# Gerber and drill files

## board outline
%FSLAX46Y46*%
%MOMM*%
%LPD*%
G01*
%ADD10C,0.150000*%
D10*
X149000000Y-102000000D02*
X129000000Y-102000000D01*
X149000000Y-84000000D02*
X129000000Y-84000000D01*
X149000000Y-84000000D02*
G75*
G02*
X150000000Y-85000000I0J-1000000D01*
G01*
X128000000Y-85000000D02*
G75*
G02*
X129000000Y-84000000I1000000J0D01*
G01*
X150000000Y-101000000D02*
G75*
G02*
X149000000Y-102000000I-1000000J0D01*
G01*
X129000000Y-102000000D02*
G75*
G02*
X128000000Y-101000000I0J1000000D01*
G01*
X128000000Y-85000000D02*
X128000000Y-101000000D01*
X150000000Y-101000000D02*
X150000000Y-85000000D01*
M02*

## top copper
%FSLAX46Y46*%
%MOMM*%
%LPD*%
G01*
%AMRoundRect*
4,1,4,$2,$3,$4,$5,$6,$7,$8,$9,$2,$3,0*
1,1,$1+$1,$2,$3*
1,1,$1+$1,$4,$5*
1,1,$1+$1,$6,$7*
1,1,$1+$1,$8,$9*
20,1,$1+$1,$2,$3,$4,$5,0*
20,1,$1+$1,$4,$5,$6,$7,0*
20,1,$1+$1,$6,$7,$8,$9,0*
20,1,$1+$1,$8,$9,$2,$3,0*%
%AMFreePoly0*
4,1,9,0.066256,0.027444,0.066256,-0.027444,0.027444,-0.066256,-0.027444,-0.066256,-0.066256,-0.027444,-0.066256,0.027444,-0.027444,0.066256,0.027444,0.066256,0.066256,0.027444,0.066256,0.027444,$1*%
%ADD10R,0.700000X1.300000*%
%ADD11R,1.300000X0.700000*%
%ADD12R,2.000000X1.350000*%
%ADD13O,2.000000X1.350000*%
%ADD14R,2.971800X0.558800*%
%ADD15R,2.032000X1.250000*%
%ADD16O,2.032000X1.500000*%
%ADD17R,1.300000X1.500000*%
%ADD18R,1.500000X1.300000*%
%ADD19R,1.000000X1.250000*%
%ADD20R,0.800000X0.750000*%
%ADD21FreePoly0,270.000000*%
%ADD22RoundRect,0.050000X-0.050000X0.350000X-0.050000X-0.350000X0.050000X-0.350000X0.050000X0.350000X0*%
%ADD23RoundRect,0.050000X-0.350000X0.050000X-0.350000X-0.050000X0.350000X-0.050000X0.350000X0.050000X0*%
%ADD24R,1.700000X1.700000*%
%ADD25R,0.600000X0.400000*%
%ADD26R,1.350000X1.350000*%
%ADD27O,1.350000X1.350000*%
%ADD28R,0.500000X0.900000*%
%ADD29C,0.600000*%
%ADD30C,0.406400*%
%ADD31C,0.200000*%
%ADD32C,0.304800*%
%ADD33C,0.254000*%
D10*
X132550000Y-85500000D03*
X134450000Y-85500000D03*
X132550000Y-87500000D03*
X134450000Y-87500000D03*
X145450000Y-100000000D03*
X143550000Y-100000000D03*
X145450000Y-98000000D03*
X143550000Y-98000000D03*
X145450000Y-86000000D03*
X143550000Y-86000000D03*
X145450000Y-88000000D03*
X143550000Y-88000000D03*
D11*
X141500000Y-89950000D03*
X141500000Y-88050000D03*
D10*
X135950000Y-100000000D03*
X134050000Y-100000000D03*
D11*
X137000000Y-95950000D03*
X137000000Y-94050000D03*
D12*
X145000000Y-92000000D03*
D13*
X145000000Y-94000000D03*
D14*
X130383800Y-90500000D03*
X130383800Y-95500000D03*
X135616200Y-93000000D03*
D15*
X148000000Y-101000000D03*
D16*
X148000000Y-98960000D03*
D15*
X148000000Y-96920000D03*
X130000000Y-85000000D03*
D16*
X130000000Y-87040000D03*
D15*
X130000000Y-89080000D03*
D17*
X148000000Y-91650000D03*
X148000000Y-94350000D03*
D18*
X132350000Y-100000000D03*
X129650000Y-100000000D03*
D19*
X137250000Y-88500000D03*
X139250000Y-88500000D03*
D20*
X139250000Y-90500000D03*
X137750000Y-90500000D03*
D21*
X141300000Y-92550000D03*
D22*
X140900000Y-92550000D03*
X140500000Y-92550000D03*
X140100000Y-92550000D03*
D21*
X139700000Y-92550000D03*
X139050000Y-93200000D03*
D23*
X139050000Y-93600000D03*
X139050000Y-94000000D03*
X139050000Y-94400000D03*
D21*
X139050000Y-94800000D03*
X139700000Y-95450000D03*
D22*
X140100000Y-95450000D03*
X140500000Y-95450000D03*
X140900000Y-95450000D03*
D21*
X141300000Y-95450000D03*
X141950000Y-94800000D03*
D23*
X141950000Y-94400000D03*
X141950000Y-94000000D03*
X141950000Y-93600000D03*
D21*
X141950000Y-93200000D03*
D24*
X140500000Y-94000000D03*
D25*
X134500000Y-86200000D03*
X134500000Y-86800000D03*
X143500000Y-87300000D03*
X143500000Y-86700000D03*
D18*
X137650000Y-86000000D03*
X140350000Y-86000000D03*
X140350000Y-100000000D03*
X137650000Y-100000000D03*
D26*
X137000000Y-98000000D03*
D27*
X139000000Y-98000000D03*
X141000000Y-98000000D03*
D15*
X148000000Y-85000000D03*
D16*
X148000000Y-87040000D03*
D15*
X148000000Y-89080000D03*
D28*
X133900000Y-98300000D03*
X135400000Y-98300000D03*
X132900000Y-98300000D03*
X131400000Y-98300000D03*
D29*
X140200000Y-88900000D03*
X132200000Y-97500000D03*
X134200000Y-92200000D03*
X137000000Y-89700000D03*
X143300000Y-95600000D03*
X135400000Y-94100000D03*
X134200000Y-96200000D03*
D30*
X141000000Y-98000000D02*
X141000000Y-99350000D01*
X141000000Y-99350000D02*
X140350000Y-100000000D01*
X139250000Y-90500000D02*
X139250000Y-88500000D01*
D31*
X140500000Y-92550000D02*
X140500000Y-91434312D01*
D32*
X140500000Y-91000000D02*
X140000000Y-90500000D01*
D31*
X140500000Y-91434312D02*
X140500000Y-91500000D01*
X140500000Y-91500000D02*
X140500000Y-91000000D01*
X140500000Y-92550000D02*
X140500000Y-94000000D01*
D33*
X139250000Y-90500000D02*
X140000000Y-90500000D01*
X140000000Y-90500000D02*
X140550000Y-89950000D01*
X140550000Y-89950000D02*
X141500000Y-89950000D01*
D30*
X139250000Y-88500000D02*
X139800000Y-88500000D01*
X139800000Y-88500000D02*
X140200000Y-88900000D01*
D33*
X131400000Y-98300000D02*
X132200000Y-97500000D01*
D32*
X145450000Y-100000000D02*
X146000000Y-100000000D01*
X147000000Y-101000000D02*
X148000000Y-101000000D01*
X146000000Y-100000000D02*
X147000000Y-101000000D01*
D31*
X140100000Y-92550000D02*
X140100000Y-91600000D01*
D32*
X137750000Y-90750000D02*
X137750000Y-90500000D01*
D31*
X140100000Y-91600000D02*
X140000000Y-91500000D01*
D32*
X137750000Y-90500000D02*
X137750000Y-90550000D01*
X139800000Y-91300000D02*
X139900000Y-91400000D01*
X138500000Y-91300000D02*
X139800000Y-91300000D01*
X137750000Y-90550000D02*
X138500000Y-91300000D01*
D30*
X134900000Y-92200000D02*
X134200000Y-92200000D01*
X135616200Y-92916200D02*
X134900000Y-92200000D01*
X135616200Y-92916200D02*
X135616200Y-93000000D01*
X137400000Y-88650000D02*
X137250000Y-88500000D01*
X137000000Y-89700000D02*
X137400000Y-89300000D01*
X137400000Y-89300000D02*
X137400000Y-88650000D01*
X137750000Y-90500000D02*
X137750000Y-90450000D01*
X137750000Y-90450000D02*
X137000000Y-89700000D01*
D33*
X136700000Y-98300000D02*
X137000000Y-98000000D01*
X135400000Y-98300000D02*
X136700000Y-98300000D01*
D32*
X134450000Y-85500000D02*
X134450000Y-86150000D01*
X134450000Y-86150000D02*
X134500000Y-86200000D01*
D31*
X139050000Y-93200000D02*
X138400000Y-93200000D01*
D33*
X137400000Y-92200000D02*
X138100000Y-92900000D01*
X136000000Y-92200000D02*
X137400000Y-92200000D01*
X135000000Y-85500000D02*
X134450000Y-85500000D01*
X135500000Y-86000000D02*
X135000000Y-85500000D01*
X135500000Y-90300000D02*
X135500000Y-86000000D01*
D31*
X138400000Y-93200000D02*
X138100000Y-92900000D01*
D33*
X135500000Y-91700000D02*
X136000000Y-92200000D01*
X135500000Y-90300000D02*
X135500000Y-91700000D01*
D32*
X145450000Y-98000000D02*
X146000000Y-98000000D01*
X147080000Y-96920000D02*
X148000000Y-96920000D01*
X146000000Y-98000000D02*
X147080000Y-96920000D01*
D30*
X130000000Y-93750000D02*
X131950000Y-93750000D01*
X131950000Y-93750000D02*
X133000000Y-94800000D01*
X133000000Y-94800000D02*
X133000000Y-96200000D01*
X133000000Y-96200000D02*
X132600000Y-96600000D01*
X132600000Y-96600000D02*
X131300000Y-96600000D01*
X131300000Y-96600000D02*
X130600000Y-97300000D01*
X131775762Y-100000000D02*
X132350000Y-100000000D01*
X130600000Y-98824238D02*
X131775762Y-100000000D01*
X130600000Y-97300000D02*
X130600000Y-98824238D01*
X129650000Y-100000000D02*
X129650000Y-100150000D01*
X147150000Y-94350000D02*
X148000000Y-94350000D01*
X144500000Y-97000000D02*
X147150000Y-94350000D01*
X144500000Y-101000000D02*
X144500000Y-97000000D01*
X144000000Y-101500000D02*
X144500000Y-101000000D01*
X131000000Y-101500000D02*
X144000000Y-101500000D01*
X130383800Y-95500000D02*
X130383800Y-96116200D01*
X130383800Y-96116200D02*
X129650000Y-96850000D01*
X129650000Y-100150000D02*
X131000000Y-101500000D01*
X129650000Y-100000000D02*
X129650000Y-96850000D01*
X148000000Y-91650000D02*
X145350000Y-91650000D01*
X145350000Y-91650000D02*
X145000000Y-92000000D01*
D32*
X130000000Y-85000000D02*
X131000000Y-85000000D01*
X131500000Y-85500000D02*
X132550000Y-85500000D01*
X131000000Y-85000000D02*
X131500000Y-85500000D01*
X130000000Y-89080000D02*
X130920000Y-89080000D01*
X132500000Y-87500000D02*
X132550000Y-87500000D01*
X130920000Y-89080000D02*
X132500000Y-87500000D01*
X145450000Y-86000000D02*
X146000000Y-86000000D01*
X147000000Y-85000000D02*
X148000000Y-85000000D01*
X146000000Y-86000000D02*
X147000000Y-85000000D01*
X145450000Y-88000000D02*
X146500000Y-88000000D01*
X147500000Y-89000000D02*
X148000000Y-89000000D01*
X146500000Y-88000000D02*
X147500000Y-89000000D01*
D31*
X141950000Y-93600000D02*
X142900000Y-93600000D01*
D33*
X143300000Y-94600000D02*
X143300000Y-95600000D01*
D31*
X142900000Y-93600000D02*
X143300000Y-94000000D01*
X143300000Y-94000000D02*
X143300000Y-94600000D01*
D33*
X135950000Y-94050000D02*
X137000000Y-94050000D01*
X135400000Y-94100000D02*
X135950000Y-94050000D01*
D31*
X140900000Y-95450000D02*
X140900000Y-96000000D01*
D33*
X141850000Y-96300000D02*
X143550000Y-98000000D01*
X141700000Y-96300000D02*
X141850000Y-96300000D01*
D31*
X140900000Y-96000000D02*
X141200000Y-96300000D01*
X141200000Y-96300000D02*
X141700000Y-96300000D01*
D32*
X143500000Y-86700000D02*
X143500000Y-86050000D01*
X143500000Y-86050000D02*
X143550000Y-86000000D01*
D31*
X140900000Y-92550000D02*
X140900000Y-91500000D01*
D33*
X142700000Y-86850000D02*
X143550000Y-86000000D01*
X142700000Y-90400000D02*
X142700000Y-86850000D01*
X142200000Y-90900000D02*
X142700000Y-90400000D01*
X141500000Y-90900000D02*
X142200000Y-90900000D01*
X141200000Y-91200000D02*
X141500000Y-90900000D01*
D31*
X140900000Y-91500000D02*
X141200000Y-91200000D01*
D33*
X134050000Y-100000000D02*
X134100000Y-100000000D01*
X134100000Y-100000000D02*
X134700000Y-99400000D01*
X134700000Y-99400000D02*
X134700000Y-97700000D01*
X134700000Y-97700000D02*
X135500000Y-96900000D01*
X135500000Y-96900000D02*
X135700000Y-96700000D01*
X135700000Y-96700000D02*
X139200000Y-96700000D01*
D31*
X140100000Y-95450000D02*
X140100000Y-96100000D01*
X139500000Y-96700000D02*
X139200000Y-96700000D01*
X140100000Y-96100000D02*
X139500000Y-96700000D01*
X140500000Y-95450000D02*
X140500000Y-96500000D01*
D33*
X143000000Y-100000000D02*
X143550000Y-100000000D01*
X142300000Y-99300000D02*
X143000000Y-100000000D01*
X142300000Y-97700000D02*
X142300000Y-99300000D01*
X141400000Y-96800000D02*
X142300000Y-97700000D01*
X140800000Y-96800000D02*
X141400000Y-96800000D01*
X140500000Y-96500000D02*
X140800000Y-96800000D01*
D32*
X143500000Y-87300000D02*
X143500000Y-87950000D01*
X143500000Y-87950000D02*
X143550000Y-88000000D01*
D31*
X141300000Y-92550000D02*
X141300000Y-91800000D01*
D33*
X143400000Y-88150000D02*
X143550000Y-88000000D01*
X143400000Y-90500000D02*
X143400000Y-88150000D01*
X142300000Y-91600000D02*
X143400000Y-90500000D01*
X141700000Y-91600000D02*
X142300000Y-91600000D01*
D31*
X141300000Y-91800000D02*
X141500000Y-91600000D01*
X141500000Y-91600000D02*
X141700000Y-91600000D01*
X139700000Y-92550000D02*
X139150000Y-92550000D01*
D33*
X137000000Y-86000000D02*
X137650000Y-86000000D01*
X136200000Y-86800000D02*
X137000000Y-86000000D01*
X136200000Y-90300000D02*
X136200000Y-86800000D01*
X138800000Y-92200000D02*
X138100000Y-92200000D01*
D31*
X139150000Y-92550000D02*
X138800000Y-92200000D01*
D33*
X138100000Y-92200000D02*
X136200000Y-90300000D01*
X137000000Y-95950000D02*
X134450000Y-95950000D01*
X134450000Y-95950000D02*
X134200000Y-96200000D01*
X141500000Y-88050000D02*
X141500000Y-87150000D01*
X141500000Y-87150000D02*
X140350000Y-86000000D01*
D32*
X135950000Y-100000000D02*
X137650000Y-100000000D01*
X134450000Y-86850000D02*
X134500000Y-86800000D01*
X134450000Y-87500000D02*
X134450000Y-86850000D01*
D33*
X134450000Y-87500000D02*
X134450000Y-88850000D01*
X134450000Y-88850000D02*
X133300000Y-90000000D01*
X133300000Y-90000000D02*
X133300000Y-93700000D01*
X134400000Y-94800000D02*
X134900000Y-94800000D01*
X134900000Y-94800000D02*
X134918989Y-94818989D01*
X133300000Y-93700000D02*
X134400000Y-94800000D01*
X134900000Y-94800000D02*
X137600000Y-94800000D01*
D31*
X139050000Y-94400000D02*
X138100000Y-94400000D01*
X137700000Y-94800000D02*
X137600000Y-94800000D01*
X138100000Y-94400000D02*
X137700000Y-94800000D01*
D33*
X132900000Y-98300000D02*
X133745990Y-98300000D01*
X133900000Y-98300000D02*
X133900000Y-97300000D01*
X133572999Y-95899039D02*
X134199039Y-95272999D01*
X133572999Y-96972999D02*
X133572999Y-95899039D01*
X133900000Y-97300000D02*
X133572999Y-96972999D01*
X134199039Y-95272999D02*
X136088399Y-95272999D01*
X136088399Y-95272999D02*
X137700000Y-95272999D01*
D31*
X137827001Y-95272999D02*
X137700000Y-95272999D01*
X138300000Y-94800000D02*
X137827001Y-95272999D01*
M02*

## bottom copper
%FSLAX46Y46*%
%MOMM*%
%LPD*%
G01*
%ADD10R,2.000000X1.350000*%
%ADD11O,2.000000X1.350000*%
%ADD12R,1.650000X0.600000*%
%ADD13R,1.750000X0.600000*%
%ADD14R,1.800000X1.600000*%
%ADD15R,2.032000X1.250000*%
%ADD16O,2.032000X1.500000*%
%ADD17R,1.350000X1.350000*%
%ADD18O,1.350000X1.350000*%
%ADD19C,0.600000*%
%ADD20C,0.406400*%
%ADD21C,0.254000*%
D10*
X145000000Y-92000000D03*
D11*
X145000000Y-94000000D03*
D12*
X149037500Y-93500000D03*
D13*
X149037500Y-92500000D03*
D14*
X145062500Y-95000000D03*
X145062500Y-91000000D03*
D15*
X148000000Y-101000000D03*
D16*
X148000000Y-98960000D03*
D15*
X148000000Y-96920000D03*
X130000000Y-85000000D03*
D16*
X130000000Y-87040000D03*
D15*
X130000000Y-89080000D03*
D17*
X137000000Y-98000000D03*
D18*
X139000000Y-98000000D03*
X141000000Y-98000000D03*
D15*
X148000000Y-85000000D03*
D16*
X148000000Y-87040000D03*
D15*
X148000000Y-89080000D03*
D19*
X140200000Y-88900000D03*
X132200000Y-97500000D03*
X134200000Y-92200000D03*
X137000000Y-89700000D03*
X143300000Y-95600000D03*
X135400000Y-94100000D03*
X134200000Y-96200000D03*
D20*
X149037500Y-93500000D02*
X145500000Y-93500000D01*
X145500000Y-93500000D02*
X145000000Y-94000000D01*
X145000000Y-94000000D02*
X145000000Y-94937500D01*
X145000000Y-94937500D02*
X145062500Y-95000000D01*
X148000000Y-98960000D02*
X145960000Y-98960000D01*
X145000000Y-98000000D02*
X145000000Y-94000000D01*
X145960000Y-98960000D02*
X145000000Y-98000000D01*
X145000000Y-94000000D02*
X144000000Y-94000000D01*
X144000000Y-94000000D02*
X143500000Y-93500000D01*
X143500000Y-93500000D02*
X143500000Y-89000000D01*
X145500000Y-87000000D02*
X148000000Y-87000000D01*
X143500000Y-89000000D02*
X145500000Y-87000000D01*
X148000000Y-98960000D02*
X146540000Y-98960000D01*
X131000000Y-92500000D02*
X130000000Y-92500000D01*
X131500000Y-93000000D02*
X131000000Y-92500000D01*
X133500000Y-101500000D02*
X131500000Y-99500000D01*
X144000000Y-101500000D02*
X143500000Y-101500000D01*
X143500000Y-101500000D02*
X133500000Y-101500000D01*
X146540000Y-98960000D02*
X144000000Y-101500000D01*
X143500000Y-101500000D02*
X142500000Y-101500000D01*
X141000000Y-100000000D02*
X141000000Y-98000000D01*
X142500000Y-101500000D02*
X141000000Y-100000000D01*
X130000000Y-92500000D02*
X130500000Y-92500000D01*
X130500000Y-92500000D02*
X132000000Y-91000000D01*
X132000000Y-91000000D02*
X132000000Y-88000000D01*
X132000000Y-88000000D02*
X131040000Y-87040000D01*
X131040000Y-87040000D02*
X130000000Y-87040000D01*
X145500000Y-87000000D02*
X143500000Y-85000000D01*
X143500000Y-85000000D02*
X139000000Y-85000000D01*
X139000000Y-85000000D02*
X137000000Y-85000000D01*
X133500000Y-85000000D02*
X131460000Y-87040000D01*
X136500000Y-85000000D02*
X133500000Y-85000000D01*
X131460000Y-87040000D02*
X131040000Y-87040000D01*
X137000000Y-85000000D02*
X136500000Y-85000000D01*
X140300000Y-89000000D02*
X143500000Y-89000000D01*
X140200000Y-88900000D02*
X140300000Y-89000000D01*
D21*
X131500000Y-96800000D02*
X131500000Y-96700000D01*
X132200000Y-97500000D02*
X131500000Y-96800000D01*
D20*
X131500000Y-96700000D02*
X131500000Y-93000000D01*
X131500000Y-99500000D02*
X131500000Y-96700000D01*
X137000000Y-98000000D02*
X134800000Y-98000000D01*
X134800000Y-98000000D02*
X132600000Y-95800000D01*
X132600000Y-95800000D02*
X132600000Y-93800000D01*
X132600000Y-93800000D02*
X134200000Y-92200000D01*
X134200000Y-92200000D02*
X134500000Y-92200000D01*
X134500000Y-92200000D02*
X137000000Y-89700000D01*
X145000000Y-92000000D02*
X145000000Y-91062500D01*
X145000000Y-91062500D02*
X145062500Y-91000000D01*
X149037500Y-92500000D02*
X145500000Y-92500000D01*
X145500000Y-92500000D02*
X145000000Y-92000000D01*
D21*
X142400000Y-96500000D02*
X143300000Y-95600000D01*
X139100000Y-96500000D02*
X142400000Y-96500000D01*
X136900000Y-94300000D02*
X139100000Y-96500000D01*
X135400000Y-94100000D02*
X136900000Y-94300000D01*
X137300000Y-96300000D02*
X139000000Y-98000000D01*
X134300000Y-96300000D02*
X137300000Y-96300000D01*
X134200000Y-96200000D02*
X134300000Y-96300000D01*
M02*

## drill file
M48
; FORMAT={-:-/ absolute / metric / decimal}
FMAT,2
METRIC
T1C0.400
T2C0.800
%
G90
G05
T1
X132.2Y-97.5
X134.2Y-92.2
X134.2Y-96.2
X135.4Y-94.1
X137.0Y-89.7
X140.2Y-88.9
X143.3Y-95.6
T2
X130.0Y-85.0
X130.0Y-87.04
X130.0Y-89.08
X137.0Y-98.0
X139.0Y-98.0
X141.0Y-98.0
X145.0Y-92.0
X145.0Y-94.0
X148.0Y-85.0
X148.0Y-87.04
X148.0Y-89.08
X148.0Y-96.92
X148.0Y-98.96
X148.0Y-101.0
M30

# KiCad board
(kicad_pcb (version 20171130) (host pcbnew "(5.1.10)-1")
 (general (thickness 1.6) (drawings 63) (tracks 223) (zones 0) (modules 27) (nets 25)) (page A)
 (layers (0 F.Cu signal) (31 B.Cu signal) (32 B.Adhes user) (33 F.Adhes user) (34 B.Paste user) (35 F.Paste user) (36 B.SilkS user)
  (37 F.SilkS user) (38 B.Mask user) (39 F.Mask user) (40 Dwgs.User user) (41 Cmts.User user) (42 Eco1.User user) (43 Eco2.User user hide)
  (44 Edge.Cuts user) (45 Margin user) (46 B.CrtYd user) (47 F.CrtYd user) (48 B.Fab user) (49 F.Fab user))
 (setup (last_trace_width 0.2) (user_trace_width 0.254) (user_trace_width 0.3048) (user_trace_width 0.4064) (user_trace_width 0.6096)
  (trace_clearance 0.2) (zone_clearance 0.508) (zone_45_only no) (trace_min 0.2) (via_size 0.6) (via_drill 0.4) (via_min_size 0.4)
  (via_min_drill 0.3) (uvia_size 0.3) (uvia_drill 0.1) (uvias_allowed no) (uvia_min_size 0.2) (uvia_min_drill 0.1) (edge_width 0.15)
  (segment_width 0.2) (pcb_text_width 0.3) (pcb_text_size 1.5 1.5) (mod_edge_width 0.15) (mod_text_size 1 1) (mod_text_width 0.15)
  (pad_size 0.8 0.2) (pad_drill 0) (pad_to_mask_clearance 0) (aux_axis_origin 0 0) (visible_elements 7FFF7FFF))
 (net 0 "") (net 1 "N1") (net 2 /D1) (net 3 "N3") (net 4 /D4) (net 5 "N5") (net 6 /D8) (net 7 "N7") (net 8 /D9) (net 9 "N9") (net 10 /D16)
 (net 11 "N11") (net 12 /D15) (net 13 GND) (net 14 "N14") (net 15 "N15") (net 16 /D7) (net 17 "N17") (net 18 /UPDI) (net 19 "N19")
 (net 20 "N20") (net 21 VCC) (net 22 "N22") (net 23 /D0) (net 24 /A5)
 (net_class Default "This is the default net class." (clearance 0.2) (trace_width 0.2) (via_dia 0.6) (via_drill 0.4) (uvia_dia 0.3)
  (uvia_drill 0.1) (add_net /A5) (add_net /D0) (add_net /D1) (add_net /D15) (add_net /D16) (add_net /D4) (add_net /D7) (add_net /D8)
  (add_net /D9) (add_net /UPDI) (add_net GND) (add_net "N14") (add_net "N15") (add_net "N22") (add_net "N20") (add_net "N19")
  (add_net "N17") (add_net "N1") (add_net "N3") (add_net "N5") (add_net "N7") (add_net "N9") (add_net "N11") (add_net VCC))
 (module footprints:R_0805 (layer F.Cu) (at 133.5 85.5 180)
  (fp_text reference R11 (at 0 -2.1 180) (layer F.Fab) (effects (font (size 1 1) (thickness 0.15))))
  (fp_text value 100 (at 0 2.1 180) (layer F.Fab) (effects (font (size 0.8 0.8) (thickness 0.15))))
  (pad 2 smd rect (at 0.95 0 180) (size 0.7 1.3) (layers F.Cu F.Paste F.Mask) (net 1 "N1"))
  (pad 1 smd rect (at -0.95 0 180) (size 0.7 1.3) (layers F.Cu F.Paste F.Mask) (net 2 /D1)))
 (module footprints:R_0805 (layer F.Cu) (at 133.5 87.5 180)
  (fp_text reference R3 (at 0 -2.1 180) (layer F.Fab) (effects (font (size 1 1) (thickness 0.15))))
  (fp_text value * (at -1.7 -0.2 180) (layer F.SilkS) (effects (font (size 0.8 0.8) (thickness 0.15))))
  (pad 2 smd rect (at 0.95 0 180) (size 0.7 1.3) (layers F.Cu F.Paste F.Mask) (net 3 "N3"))
  (pad 1 smd rect (at -0.95 0 180) (size 0.7 1.3) (layers F.Cu F.Paste F.Mask) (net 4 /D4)))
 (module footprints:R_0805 (layer F.Cu) (at 144.5 100)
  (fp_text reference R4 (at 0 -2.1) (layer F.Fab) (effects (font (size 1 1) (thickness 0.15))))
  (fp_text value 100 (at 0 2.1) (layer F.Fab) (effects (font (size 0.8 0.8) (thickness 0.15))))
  (pad 2 smd rect (at 0.95 0) (size 0.7 1.3) (layers F.Cu F.Paste F.Mask) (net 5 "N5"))
  (pad 1 smd rect (at -0.95 0) (size 0.7 1.3) (layers F.Cu F.Paste F.Mask) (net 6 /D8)))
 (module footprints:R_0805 (layer F.Cu) (at 144.5 98)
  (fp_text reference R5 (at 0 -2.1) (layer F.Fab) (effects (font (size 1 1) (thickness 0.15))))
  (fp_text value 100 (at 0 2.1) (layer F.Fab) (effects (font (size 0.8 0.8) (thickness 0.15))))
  (pad 2 smd rect (at 0.95 0) (size 0.7 1.3) (layers F.Cu F.Paste F.Mask) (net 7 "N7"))
  (pad 1 smd rect (at -0.95 0) (size 0.7 1.3) (layers F.Cu F.Paste F.Mask) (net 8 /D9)))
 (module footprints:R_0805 (layer F.Cu) (at 144.5 86)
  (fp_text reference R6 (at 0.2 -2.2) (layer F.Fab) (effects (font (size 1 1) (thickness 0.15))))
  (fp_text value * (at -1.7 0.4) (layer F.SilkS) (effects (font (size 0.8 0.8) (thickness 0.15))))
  (pad 2 smd rect (at 0.95 0) (size 0.7 1.3) (layers F.Cu F.Paste F.Mask) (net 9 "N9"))
  (pad 1 smd rect (at -0.95 0) (size 0.7 1.3) (layers F.Cu F.Paste F.Mask) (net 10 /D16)))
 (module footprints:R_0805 (layer F.Cu) (at 144.5 88)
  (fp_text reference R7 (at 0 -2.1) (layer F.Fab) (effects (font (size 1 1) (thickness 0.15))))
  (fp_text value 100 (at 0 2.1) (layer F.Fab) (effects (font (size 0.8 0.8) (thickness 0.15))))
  (pad 2 smd rect (at 0.95 0) (size 0.7 1.3) (layers F.Cu F.Paste F.Mask) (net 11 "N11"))
  (pad 1 smd rect (at -0.95 0) (size 0.7 1.3) (layers F.Cu F.Paste F.Mask) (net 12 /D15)))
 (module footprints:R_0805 (layer F.Cu) (at 141.5 89 270)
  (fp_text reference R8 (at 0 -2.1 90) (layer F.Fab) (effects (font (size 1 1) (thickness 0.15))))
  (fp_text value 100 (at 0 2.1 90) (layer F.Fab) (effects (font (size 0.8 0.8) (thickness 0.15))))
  (pad 2 smd rect (at 0.95 0 270) (size 0.7 1.3) (layers F.Cu F.Paste F.Mask) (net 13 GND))
  (pad 1 smd rect (at -0.95 0 270) (size 0.7 1.3) (layers F.Cu F.Paste F.Mask) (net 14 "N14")))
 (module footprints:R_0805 (layer F.Cu) (at 135 100)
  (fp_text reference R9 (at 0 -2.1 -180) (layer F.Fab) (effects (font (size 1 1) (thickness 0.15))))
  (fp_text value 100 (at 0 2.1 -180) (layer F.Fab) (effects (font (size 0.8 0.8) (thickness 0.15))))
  (pad 2 smd rect (at 0.95 0) (size 0.7 1.3) (layers F.Cu F.Paste F.Mask) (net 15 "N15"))
  (pad 1 smd rect (at -0.95 0) (size 0.7 1.3) (layers F.Cu F.Paste F.Mask) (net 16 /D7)))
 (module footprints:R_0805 (layer F.Cu) (at 137 95 270)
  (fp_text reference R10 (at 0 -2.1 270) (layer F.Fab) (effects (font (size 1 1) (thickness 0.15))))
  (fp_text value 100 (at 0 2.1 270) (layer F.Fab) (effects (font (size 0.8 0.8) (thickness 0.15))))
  (pad 2 smd rect (at 0.95 0 270) (size 0.7 1.3) (layers F.Cu F.Paste F.Mask) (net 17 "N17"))
  (pad 1 smd rect (at -0.95 0 270) (size 0.7 1.3) (layers F.Cu F.Paste F.Mask) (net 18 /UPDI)))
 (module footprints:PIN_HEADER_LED (layer B.Cu) (at 145 92 180)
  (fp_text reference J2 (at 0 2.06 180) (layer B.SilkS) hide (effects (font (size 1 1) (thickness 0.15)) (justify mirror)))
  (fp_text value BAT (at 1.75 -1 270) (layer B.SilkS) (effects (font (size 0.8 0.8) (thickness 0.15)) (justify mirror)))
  (pad 1 thru_hole rect (at 0 0 180) (size 2 1.35) (drill 0.8) (layers *.Cu *.Mask) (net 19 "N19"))
  (pad 2 thru_hole oval (at 0 -2 180) (size 2 1.35) (drill 0.8) (layers *.Cu *.Mask) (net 13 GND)))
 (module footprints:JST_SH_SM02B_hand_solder (layer B.Cu) (at 147 93 90)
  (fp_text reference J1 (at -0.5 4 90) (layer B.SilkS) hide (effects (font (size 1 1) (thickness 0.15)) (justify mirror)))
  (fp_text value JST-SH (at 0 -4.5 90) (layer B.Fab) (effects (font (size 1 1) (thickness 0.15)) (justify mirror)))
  (pad 1 smd rect (at -0.5 2.0375 90) (size 0.6 1.65) (layers B.Cu B.Paste B.Mask) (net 13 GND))
  (pad 2 smd rect (at 0.5 2.0375 90) (size 0.6 1.75) (layers B.Cu B.Paste B.Mask) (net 19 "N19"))
  (pad 1 smd rect (at -2 -1.9375 90) (size 1.6 1.8) (layers B.Cu B.Paste B.Mask) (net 13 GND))
  (pad 2 smd rect (at 2 -1.9375 90) (size 1.6 1.8) (layers B.Cu B.Paste B.Mask) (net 19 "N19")))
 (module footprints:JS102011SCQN (layer F.Cu) (at 133 93)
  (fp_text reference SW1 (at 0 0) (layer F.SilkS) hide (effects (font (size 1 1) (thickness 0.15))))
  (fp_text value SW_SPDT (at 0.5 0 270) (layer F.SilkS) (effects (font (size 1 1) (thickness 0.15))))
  (pad 1 smd rect (at -2.6162 -2.5) (size 2.9718 0.5588) (layers F.Cu F.Paste F.Mask))
  (pad 3 smd rect (at -2.6162 2.5) (size 2.9718 0.5588) (layers F.Cu F.Paste F.Mask) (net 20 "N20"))
  (pad 2 smd rect (at 2.6162 0) (size 2.9718 0.5588) (layers F.Cu F.Paste F.Mask) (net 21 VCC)))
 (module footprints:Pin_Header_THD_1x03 (layer F.Cu) (at 148 101 180)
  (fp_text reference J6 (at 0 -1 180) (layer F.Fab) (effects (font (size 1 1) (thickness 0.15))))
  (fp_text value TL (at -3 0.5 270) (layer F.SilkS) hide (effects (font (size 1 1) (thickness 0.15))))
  (pad 1 thru_hole rect (at 0 0 180) (size 2.032 1.25) (drill 0.8) (layers *.Cu *.Mask F.SilkS) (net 5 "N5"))
  (pad 2 thru_hole oval (at 0 2.04 180) (size 2.032 1.5) (drill 0.8) (layers *.Cu *.Mask F.SilkS) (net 13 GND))
  (pad 3 thru_hole rect (at 0 4.08 180) (size 2.032 1.25) (drill 0.8) (layers *.Cu *.Mask F.SilkS) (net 7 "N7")))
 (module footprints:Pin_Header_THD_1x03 (layer F.Cu) (at 130 85)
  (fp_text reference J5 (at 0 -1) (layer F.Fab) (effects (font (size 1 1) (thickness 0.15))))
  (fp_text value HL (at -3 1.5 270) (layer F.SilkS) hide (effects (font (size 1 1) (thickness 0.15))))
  (pad 1 thru_hole rect (at 0 0) (size 2.032 1.25) (drill 0.8) (layers *.Cu *.Mask F.SilkS) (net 1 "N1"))
  (pad 2 thru_hole oval (at 0 2.04) (size 2.032 1.5) (drill 0.8) (layers *.Cu *.Mask F.SilkS) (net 13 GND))
  (pad 3 thru_hole rect (at 0 4.08) (size 2.032 1.25) (drill 0.8) (layers *.Cu *.Mask F.SilkS) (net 3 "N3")))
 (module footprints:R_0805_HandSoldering (layer F.Cu) (at 148 93 270)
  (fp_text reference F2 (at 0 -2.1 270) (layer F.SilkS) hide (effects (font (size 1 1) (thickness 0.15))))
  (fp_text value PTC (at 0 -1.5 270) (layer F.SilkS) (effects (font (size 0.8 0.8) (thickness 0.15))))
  (pad 1 smd rect (at -1.35 0 270) (size 1.5 1.3) (layers F.Cu F.Paste F.Mask) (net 19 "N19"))
  (pad 2 smd rect (at 1.35 0 270) (size 1.5 1.3) (layers F.Cu F.Paste F.Mask) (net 20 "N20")))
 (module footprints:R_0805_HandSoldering (layer F.Cu) (at 131 100 180)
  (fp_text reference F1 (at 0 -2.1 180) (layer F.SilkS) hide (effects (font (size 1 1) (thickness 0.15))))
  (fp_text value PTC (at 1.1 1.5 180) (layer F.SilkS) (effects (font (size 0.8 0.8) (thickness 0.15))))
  (pad 1 smd rect (at -1.35 0 180) (size 1.5 1.3) (layers F.Cu F.Paste F.Mask) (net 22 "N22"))
  (pad 2 smd rect (at 1.35 0 180) (size 1.5 1.3) (layers F.Cu F.Paste F.Mask) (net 20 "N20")))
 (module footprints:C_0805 (layer F.Cu) (at 138.25 88.5)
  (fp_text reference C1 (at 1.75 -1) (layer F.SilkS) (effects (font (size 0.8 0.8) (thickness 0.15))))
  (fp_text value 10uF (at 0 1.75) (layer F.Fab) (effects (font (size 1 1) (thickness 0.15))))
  (pad 1 smd rect (at -1 0) (size 1 1.25) (layers F.Cu F.Paste F.Mask) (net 21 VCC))
  (pad 2 smd rect (at 1 0) (size 1 1.25) (layers F.Cu F.Paste F.Mask) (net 13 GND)))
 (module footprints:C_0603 (layer F.Cu) (at 138.5 90.5)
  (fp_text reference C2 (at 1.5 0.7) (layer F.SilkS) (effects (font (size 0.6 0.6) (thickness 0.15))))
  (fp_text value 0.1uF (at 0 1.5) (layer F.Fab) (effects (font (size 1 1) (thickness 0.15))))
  (pad 2 smd rect (at 0.75 0) (size 0.8 0.75) (layers F.Cu F.Paste F.Mask) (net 13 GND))
  (pad 1 smd rect (at -0.75 0) (size 0.8 0.75) (layers F.Cu F.Paste F.Mask) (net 21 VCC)))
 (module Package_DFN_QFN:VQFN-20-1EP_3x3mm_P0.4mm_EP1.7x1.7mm (layer F.Cu) (at 140.5 94 270)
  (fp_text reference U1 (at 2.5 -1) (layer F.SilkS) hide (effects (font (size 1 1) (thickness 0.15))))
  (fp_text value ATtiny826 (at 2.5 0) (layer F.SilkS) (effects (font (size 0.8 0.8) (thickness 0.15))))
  (pad 1 smd custom (at -1.45 -0.8 270) (size 0.143431 0.143431) (layers F.Cu F.Paste F.Mask) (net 12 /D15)
   (options (clearance outline) (anchor circle)) (primitives))
  (pad 2 smd roundrect (at -1.45 -0.4 270) (size 0.8 0.2) (layers F.Cu F.Paste F.Mask) (roundrect_rratio 0.25) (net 10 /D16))
  (pad 3 smd roundrect (at -1.45 0 270) (size 0.8 0.2) (layers F.Cu F.Paste F.Mask) (roundrect_rratio 0.25) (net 13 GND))
  (pad 4 smd roundrect (at -1.45 0.4 270) (size 0.8 0.2) (layers F.Cu F.Paste F.Mask) (roundrect_rratio 0.25) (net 21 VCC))
  (pad 5 smd custom (at -1.45 0.8 270) (size 0.143431 0.143431) (layers F.Cu F.Paste F.Mask) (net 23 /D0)
   (options (clearance outline) (anchor circle)) (primitives))
  (pad 6 smd custom (at -0.8 1.45 270) (size 0.143431 0.143431) (layers F.Cu F.Paste F.Mask) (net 2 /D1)
   (options (clearance outline) (anchor circle)) (primitives))
  (pad 7 smd roundrect (at -0.4 1.45 270) (size 0.2 0.8) (layers F.Cu F.Paste F.Mask) (roundrect_rratio 0.25))
  (pad 8 smd roundrect (at 0 1.45 270) (size 0.2 0.8) (layers F.Cu F.Paste F.Mask) (roundrect_rratio 0.25))
  (pad 9 smd roundrect (at 0.4 1.45 270) (size 0.2 0.8) (layers F.Cu F.Paste F.Mask) (roundrect_rratio 0.25) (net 4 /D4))
  (pad 10 smd custom (at 0.8 1.45 270) (size 0.143431 0.143431) (layers F.Cu F.Paste F.Mask) (options (clearance outline) (anchor circle))
   (primitives))
  (pad 11 smd custom (at 1.45 0.8 270) (size 0.143431 0.143431) (layers F.Cu F.Paste F.Mask) (options (clearance outline) (anchor circle))
   (primitives))
  (pad 12 smd roundrect (at 1.45 0.4 270) (size 0.8 0.2) (layers F.Cu F.Paste F.Mask) (roundrect_rratio 0.25) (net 16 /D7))
  (pad 13 smd roundrect (at 1.45 0 270) (size 0.8 0.2) (layers F.Cu F.Paste F.Mask) (roundrect_rratio 0.25) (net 6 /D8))
  (pad 14 smd roundrect (at 1.45 -0.4 270) (size 0.8 0.2) (layers F.Cu F.Paste F.Mask) (roundrect_rratio 0.25) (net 8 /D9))
  (pad 15 smd custom (at 1.45 -0.8 270) (size 0.143431 0.143431) (layers F.Cu F.Paste F.Mask) (options (clearance outline) (anchor circle))
   (primitives))
  (pad 16 smd custom (at 0.8 -1.45 270) (size 0.143431 0.143431) (layers F.Cu F.Paste F.Mask) (options (clearance outline) (anchor circle))
   (primitives))
  (pad 17 smd roundrect (at 0.4 -1.45 270) (size 0.2 0.8) (layers F.Cu F.Paste F.Mask) (roundrect_rratio 0.25))
  (pad 18 smd roundrect (at 0 -1.45 270) (size 0.2 0.8) (layers F.Cu F.Paste F.Mask) (roundrect_rratio 0.25))
  (pad 19 smd roundrect (at -0.4 -1.45 270) (size 0.2 0.8) (layers F.Cu F.Paste F.Mask) (roundrect_rratio 0.25) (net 18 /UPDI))
  (pad 20 smd custom (at -0.8 -1.45 270) (size 0.143431 0.143431) (layers F.Cu F.Paste F.Mask) (options (clearance outline) (anchor circle))
   (primitives))
  (pad 21 smd rect (at 0 0 270) (size 1.7 1.7) (layers F.Cu F.Mask) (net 13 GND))
  (pad "" smd roundrect (at -0.425 -0.425 270) (size 0.69 0.69) (layers F.Paste) (roundrect_rratio 0.25))
  (pad "" smd roundrect (at -0.425 0.425 270) (size 0.69 0.69) (layers F.Paste) (roundrect_rratio 0.25))
  (pad "" smd roundrect (at 0.425 -0.425 270) (size 0.69 0.69) (layers F.Paste) (roundrect_rratio 0.25))
  (pad "" smd roundrect (at 0.425 0.425 270) (size 0.69 0.69) (layers F.Paste) (roundrect_rratio 0.25)))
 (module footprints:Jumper (layer F.Cu) (at 134.5 86.5 270)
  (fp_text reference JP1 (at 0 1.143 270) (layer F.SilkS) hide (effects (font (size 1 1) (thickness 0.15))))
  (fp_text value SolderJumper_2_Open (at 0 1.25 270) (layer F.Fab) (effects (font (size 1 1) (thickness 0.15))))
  (pad 1 smd rect (at -0.3 0 270) (size 0.4 0.6) (layers F.Cu F.Paste F.Mask) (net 2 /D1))
  (pad 2 smd rect (at 0.3 0 270) (size 0.4 0.6) (layers F.Cu F.Paste F.Mask) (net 4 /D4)))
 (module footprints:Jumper (layer F.Cu) (at 143.5 87 270)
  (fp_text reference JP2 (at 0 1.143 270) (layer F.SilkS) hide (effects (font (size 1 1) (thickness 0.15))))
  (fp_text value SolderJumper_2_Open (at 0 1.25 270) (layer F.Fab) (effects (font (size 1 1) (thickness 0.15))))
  (pad 2 smd rect (at 0.3 0 270) (size 0.4 0.6) (layers F.Cu F.Paste F.Mask) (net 12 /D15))
  (pad 1 smd rect (at -0.3 0 270) (size 0.4 0.6) (layers F.Cu F.Paste F.Mask) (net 10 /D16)))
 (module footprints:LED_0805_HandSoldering (layer F.Cu) (at 139 86 180)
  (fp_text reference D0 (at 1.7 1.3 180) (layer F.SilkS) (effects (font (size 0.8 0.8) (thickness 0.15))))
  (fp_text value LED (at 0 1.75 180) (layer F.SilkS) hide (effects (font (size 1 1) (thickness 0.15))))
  (pad 2 smd rect (at 1.35 0 180) (size 1.5 1.3) (layers F.Cu F.Paste F.Mask) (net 23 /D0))
  (pad 1 smd rect (at -1.35 0 180) (size 1.5 1.3) (layers F.Cu F.Paste F.Mask) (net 14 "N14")))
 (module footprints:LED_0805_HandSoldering (layer F.Cu) (at 139 100 180)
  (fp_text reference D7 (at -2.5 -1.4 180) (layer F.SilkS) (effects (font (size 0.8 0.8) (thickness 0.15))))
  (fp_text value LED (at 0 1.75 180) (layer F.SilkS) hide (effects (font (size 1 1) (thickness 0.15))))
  (pad 1 smd rect (at -1.35 0 180) (size 1.5 1.3) (layers F.Cu F.Paste F.Mask) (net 13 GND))
  (pad 2 smd rect (at 1.35 0 180) (size 1.5 1.3) (layers F.Cu F.Paste F.Mask) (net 15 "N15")))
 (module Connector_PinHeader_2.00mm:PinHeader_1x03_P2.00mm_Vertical (layer B.Cu) (at 137 98 270)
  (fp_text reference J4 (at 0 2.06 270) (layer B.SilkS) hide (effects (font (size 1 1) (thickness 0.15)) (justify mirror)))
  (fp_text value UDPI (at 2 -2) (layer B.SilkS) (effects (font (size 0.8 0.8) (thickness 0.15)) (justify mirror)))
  (pad 1 thru_hole rect (at 0 0 270) (size 1.35 1.35) (drill 0.8) (layers *.Cu *.Mask) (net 21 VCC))
  (pad 2 thru_hole oval (at 0 -2 270) (size 1.35 1.35) (drill 0.8) (layers *.Cu *.Mask) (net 17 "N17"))
  (pad 3 thru_hole oval (at 0 -4 270) (size 1.35 1.35) (drill 0.8) (layers *.Cu *.Mask) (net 13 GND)))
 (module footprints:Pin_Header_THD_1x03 (layer F.Cu) (at 148 85)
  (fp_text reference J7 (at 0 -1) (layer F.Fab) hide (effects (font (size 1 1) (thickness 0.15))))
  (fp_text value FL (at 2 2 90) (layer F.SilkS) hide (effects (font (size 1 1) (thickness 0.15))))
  (pad 1 thru_hole rect (at 0 0) (size 2.032 1.25) (drill 0.8) (layers *.Cu *.Mask F.SilkS) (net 9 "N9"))
  (pad 2 thru_hole oval (at 0 2.04) (size 2.032 1.5) (drill 0.8) (layers *.Cu *.Mask F.SilkS) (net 13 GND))
  (pad 3 thru_hole rect (at 0 4.08) (size 2.032 1.25) (drill 0.8) (layers *.Cu *.Mask F.SilkS) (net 11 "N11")))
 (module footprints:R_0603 (layer F.Cu) (at 134.65 98.3 180)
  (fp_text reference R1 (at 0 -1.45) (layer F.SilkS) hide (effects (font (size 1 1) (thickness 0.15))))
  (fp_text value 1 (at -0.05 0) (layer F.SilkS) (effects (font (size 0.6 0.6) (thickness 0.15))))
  (pad 2 smd rect (at 0.75 0 180) (size 0.5 0.9) (layers F.Cu F.Paste F.Mask) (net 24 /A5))
  (pad 1 smd rect (at -0.75 0 180) (size 0.5 0.9) (layers F.Cu F.Paste F.Mask) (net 21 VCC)))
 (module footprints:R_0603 (layer F.Cu) (at 132.15 98.3 180)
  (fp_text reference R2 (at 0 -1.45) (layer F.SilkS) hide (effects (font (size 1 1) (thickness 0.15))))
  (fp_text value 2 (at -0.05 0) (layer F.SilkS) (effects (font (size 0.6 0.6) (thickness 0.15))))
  (pad 1 smd rect (at -0.75 0 180) (size 0.5 0.9) (layers F.Cu F.Paste F.Mask) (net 24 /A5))
  (pad 2 smd rect (at 0.75 0 180) (size 0.5 0.9) (layers F.Cu F.Paste F.Mask) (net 13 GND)))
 (gr_line (start 149 102) (end 129 102) (angle 90) (layer Edge.Cuts) (width 0.15))
 (gr_line (start 149 84) (end 129 84) (angle 90) (layer Edge.Cuts) (width 0.15))
 (gr_arc (start 149 85) (end 149 84) (angle 90) (layer Edge.Cuts) (width 0.15))
 (gr_arc (start 129 85) (end 128 85) (angle 90) (layer Edge.Cuts) (width 0.15))
 (gr_arc (start 149 101) (end 150 101) (angle 90) (layer Edge.Cuts) (width 0.15))
 (gr_arc (start 129 101) (end 129 102) (angle 90) (layer Edge.Cuts) (width 0.15))
 (gr_line (start 128 85) (end 128 101) (angle 90) (layer Edge.Cuts) (width 0.15))
 (gr_line (start 150 101) (end 150 85) (angle 90) (layer Edge.Cuts) (width 0.15))
 (segment (start 149.0375 93.5) (end 145.5 93.5) (width 0.4064) (layer B.Cu) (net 13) (status C00030))
 (segment (start 145.5 93.5) (end 145 94) (width 0.4064) (layer B.Cu) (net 13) (status C00030))
 (segment (start 145 94) (end 145 94.9375) (width 0.4064) (layer B.Cu) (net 13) (status C00030))
 (segment (start 145 94.9375) (end 145.0625 95) (width 0.4064) (layer B.Cu) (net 13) (status C00030))
 (segment (start 148 98.96) (end 145.96 98.96) (width 0.4064) (layer B.Cu) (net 13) (status 400010))
 (segment (start 145 98) (end 145 94) (width 0.4064) (layer B.Cu) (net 13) (status 800020))
 (segment (start 145.96 98.96) (end 145 98) (width 0.4064) (layer B.Cu) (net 13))
 (segment (start 145 94) (end 144 94) (width 0.4064) (layer B.Cu) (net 13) (status C00030))
 (segment (start 144 94) (end 143.5 93.5) (width 0.4064) (layer B.Cu) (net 13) (status 400010))
 (segment (start 143.5 93.5) (end 143.5 89) (width 0.4064) (layer B.Cu) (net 13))
 (segment (start 145.5 87) (end 148 87) (width 0.4064) (layer B.Cu) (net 13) (status 800020))
 (segment (start 143.5 89) (end 145.5 87) (width 0.4064) (layer B.Cu) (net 13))
 (segment (start 148 98.96) (end 146.54 98.96) (width 0.4064) (layer B.Cu) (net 13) (status 400010))
 (segment (start 131 92.5) (end 130 92.5) (width 0.4064) (layer B.Cu) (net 13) (status 800020))
 (segment (start 131.5 93) (end 131 92.5) (width 0.4064) (layer B.Cu) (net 13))
 (segment (start 133.5 101.5) (end 131.5 99.5) (width 0.4064) (layer B.Cu) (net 13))
 (segment (start 144 101.5) (end 143.5 101.5) (width 0.4064) (layer B.Cu) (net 13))
 (segment (start 143.5 101.5) (end 133.5 101.5) (width 0.4064) (layer B.Cu) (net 13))
 (segment (start 146.54 98.96) (end 144 101.5) (width 0.4064) (layer B.Cu) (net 13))
 (segment (start 143.5 101.5) (end 142.5 101.5) (width 0.4064) (layer B.Cu) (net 13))
 (segment (start 141 100) (end 141 98) (width 0.4064) (layer B.Cu) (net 13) (status 800020))
 (segment (start 142.5 101.5) (end 141 100) (width 0.4064) (layer B.Cu) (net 13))
 (segment (start 141 98) (end 141 99.35) (width 0.4064) (layer F.Cu) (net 13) (status C00030))
 (segment (start 141 99.35) (end 140.35 100) (width 0.4064) (layer F.Cu) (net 13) (status C00030))
 (segment (start 130 92.5) (end 130.5 92.5) (width 0.4064) (layer B.Cu) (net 13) (status C00030))
 (segment (start 130.5 92.5) (end 132 91) (width 0.4064) (layer B.Cu) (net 13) (status 400010))
 (segment (start 132 91) (end 132 88) (width 0.4064) (layer B.Cu) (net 13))
 (segment (start 132 88) (end 131.04 87.04) (width 0.4064) (layer B.Cu) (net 13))
 (segment (start 131.04 87.04) (end 130 87.04) (width 0.4064) (layer B.Cu) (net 13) (status 800020))
 (segment (start 145.5 87) (end 143.5 85) (width 0.4064) (layer B.Cu) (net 13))
 (segment (start 143.5 85) (end 139 85) (width 0.4064) (layer B.Cu) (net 13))
 (segment (start 139 85) (end 137 85) (width 0.4064) (layer B.Cu) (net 13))
 (segment (start 133.5 85) (end 131.46 87.04) (width 0.4064) (layer B.Cu) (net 13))
 (segment (start 136.5 85) (end 133.5 85) (width 0.4064) (layer B.Cu) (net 13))
 (segment (start 131.46 87.04) (end 131.04 87.04) (width 0.4064) (layer B.Cu) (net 13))
 (segment (start 137 85) (end 136.5 85) (width 0.4064) (layer B.Cu) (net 13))
 (segment (start 139.25 90.5) (end 139.25 88.5) (width 0.4064) (layer F.Cu) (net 13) (status C00030))
 (segment (start 140.5 92.55) (end 140.5 91.434312) (width 0.2) (layer F.Cu) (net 13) (status 400010))
 (segment (start 140.5 91) (end 140 90.5) (width 0.3048) (layer F.Cu) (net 13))
 (segment (start 140.5 91.434312) (end 140.5 91.5) (width 0.2) (layer F.Cu) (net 13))
 (segment (start 140.5 91.5) (end 140.5 91) (width 0.2) (layer F.Cu) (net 13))
 (segment (start 140.5 92.55) (end 140.5 94) (width 0.2) (layer F.Cu) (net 13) (status C00030))
 (segment (start 139.25 90.5) (end 140 90.5) (width 0.254) (layer F.Cu) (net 13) (status 400010))
 (segment (start 140 90.5) (end 140.55 89.95) (width 0.254) (layer F.Cu) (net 13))
 (segment (start 140.55 89.95) (end 141.5 89.95) (width 0.254) (layer F.Cu) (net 13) (status 800020))
 (segment (start 139.25 88.5) (end 139.8 88.5) (width 0.4064) (layer F.Cu) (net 13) (status 400010))
 (segment (start 140.3 89) (end 143.5 89) (width 0.4064) (layer B.Cu) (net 13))
 (segment (start 140.2 88.9) (end 140.3 89) (width 0.4064) (layer B.Cu) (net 13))
 (via (at 140.2 88.9) (size 0.6) (drill 0.4) (layers F.Cu B.Cu) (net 13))
 (segment (start 139.8 88.5) (end 140.2 88.9) (width 0.4064) (layer F.Cu) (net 13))
 (via (at 132.2 97.5) (size 0.6) (drill 0.4) (layers F.Cu B.Cu) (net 13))
 (segment (start 131.4 98.3) (end 132.2 97.5) (width 0.254) (layer F.Cu) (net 13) (status 10))
 (segment (start 131.5 96.8) (end 131.5 96.7) (width 0.254) (layer B.Cu) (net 13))
 (segment (start 132.2 97.5) (end 131.5 96.8) (width 0.254) (layer B.Cu) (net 13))
 (segment (start 131.5 96.7) (end 131.5 93) (width 0.4064) (layer B.Cu) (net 13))
 (segment (start 131.5 99.5) (end 131.5 96.7) (width 0.4064) (layer B.Cu) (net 13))
 (segment (start 145.45 100) (end 146 100) (width 0.3048) (layer F.Cu) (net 5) (status 400010))
 (segment (start 147 101) (end 148 101) (width 0.3048) (layer F.Cu) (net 5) (status C00030))
 (segment (start 146 100) (end 147 101) (width 0.3048) (layer F.Cu) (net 5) (status 800020))
 (segment (start 140.1 92.55) (end 140.1 91.6) (width 0.2) (layer F.Cu) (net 21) (status 400010))
 (segment (start 137.75 90.75) (end 137.75 90.5) (width 0.3048) (layer F.Cu) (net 21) (status C00030))
 (segment (start 140.1 91.6) (end 140 91.5) (width 0.2) (layer F.Cu) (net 21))
 (segment (start 137.75 90.5) (end 137.75 90.55) (width 0.3048) (layer F.Cu) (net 21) (status C00030))
 (segment (start 139.8 91.3) (end 139.9 91.4) (width 0.3048) (layer F.Cu) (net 21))
 (segment (start 138.5 91.3) (end 139.8 91.3) (width 0.3048) (layer F.Cu) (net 21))
 (segment (start 137.75 90.55) (end 138.5 91.3) (width 0.3048) (layer F.Cu) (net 21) (status 400010))
 (segment (start 137 98) (end 134.8 98) (width 0.4064) (layer B.Cu) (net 21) (status 400010))
 (segment (start 134.9 92.2) (end 134.2 92.2) (width 0.4064) (layer F.Cu) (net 21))
 (segment (start 135.6162 92.9162) (end 134.9 92.2) (width 0.4064) (layer F.Cu) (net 21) (status 400010))
 (segment (start 135.6162 92.9162) (end 135.6162 93) (width 0.4064) (layer F.Cu) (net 21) (status C00030))
 (segment (start 134.8 98) (end 132.6 95.8) (width 0.4064) (layer B.Cu) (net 21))
 (segment (start 132.6 95.8) (end 132.6 93.8) (width 0.4064) (layer B.Cu) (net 21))
 (segment (start 132.6 93.8) (end 134.2 92.2) (width 0.4064) (layer B.Cu) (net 21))
 (via (at 134.2 92.2) (size 0.6) (drill 0.4) (layers F.Cu B.Cu) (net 21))
 (segment (start 134.2 92.2) (end 134.5 92.2) (width 0.4064) (layer B.Cu) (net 21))
 (via (at 137 89.7) (size 0.6) (drill 0.4) (layers F.Cu B.Cu) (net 21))
 (segment (start 134.5 92.2) (end 137 89.7) (width 0.4064) (layer B.Cu) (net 21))
 (segment (start 137.4 88.65) (end 137.25 88.5) (width 0.4064) (layer F.Cu) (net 21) (status C00030))
 (segment (start 137 89.7) (end 137.4 89.3) (width 0.4064) (layer F.Cu) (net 21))
 (segment (start 137.4 89.3) (end 137.4 88.65) (width 0.4064) (layer F.Cu) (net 21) (status 800020))
 (segment (start 137.75 90.5) (end 137.75 90.45) (width 0.4064) (layer F.Cu) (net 21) (status C00030))
 (segment (start 137.75 90.45) (end 137 89.7) (width 0.4064) (layer F.Cu) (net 21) (status 400010))
 (segment (start 136.7 98.3) (end 137 98) (width 0.254) (layer F.Cu) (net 21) (status 30))
 (segment (start 135.4 98.3) (end 136.7 98.3) (width 0.254) (layer F.Cu) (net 21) (status 30))
 (segment (start 134.45 85.5) (end 134.45 86.15) (width 0.3048) (layer F.Cu) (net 2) (status C00030))
 (segment (start 134.45 86.15) (end 134.5 86.2) (width 0.3048) (layer F.Cu) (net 2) (status C00030))
 (segment (start 139.05 93.2) (end 138.4 93.2) (width 0.2) (layer F.Cu) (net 2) (status 400010))
 (segment (start 137.4 92.2) (end 138.1 92.9) (width 0.254) (layer F.Cu) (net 2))
 (segment (start 136 92.2) (end 137.4 92.2) (width 0.254) (layer F.Cu) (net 2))
 (segment (start 135 85.5) (end 134.45 85.5) (width 0.254) (layer F.Cu) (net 2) (status 800020))
 (segment (start 135.5 86) (end 135 85.5) (width 0.254) (layer F.Cu) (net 2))
 (segment (start 135.5 90.3) (end 135.5 86) (width 0.254) (layer F.Cu) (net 2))
 (segment (start 138.4 93.2) (end 138.1 92.9) (width 0.2) (layer F.Cu) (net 2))
 (segment (start 135.5 91.7) (end 136 92.2) (width 0.254) (layer F.Cu) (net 2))
 (segment (start 135.5 90.3) (end 135.5 91.7) (width 0.254) (layer F.Cu) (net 2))
 (segment (start 145.45 98) (end 146 98) (width 0.3048) (layer F.Cu) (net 7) (status 400010))
 (segment (start 147.08 96.92) (end 148 96.92) (width 0.3048) (layer F.Cu) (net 7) (status C00030))
 (segment (start 146 98) (end 147.08 96.92) (width 0.3048) (layer F.Cu) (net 7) (status 800020))
 (segment (start 130 93.75) (end 131.95 93.75) (width 0.4064) (layer F.Cu) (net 22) (status 10))
 (segment (start 131.95 93.75) (end 133 94.8) (width 0.4064) (layer F.Cu) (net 22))
 (segment (start 133 94.8) (end 133 96.2) (width 0.4064) (layer F.Cu) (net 22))
 (segment (start 133 96.2) (end 132.6 96.6) (width 0.4064) (layer F.Cu) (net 22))
 (segment (start 132.6 96.6) (end 131.3 96.6) (width 0.4064) (layer F.Cu) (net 22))
 (segment (start 131.3 96.6) (end 130.6 97.3) (width 0.4064) (layer F.Cu) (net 22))
 (segment (start 131.775762 100) (end 132.35 100) (width 0.4064) (layer F.Cu) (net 22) (status 30))
 (segment (start 130.6 98.824238) (end 131.775762 100) (width 0.4064) (layer F.Cu) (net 22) (status 20))
 (segment (start 130.6 97.3) (end 130.6 98.824238) (width 0.4064) (layer F.Cu) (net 22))
 (segment (start 129.65 100) (end 129.65 100.15) (width 0.4064) (layer F.Cu) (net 20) (status C00030))
 (segment (start 147.15 94.35) (end 148 94.35) (width 0.4064) (layer F.Cu) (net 20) (status 800020))
 (segment (start 144.5 97) (end 147.15 94.35) (width 0.4064) (layer F.Cu) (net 20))
 (segment (start 144.5 101) (end 144.5 97) (width 0.4064) (layer F.Cu) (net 20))
 (segment (start 144 101.5) (end 144.5 101) (width 0.4064) (layer F.Cu) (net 20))
 (segment (start 131 101.5) (end 144 101.5) (width 0.4064) (layer F.Cu) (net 20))
 (segment (start 130.3838 95.5) (end 130.3838 96.1162) (width 0.4064) (layer F.Cu) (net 20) (status 400010))
 (segment (start 130.3838 96.1162) (end 129.65 96.85) (width 0.4064) (layer F.Cu) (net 20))
 (segment (start 129.65 100.15) (end 131 101.5) (width 0.4064) (layer F.Cu) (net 20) (status 400010))
 (segment (start 129.65 100) (end 129.65 96.85) (width 0.4064) (layer F.Cu) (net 20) (status 10))
 (segment (start 148 91.65) (end 145.35 91.65) (width 0.4064) (layer F.Cu) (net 19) (status C00030))
 (segment (start 145.35 91.65) (end 145 92) (width 0.4064) (layer F.Cu) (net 19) (status C00030))
 (segment (start 145 92) (end 145 91.0625) (width 0.4064) (layer B.Cu) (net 19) (status C00030))
 (segment (start 145 91.0625) (end 145.0625 91) (width 0.4064) (layer B.Cu) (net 19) (status C00030))
 (segment (start 149.0375 92.5) (end 145.5 92.5) (width 0.4064) (layer B.Cu) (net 19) (status C00030))
 (segment (start 145.5 92.5) (end 145 92) (width 0.4064) (layer B.Cu) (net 19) (status C00030))
 (segment (start 130 85) (end 131 85) (width 0.3048) (layer F.Cu) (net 1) (status C00030))
 (segment (start 131.5 85.5) (end 132.55 85.5) (width 0.3048) (layer F.Cu) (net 1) (status 800020))
 (segment (start 131 85) (end 131.5 85.5) (width 0.3048) (layer F.Cu) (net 1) (status 400010))
 (segment (start 130 89.08) (end 130.92 89.08) (width 0.3048) (layer F.Cu) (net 3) (status C00030))
 (segment (start 132.5 87.5) (end 132.55 87.5) (width 0.3048) (layer F.Cu) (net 3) (status C00030))
 (segment (start 130.92 89.08) (end 132.5 87.5) (width 0.3048) (layer F.Cu) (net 3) (status C00030))
 (segment (start 145.45 86) (end 146 86) (width 0.3048) (layer F.Cu) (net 9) (status 400010))
 (segment (start 147 85) (end 148 85) (width 0.3048) (layer F.Cu) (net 9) (status 800030))
 (segment (start 146 86) (end 147 85) (width 0.3048) (layer F.Cu) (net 9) (status 20))
 (segment (start 145.45 88) (end 146.5 88) (width 0.3048) (layer F.Cu) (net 11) (status 400010))
 (segment (start 147.5 89) (end 148 89) (width 0.3048) (layer F.Cu) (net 11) (status C00030))
 (segment (start 146.5 88) (end 147.5 89) (width 0.3048) (layer F.Cu) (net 11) (status 800020))
 (segment (start 141.95 93.6) (end 142.9 93.6) (width 0.2) (layer F.Cu) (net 18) (status 400010))
 (via (at 143.3 95.6) (size 0.6) (drill 0.4) (layers F.Cu B.Cu) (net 18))
 (segment (start 143.3 94.6) (end 143.3 95.6) (width 0.254) (layer F.Cu) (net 18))
 (segment (start 142.9 93.6) (end 143.3 94) (width 0.2) (layer F.Cu) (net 18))
 (segment (start 143.3 94) (end 143.3 94.6) (width 0.2) (layer F.Cu) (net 18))
 (segment (start 142.4 96.5) (end 143.3 95.6) (width 0.254) (layer B.Cu) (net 18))
 (segment (start 139.1 96.5) (end 142.4 96.5) (width 0.254) (layer B.Cu) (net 18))
 (segment (start 136.9 94.3) (end 139.1 96.5) (width 0.254) (layer B.Cu) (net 18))
 (segment (start 135.95 94.05) (end 137 94.05) (width 0.254) (layer F.Cu) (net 18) (status 20))
 (segment (start 135.4 94.1) (end 136.9 94.3) (width 0.254) (layer B.Cu) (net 18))
 (segment (start 135.4 94.1) (end 135.95 94.05) (width 0.254) (layer F.Cu) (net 18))
 (via (at 135.4 94.1) (size 0.6) (drill 0.4) (layers F.Cu B.Cu) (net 18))
 (segment (start 140.9 95.45) (end 140.9 96) (width 0.2) (layer F.Cu) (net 8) (status 400010))
 (segment (start 141.85 96.3) (end 143.55 98) (width 0.254) (layer F.Cu) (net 8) (status 800020))
 (segment (start 141.7 96.3) (end 141.85 96.3) (width 0.254) (layer F.Cu) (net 8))
 (segment (start 140.9 96) (end 141.2 96.3) (width 0.2) (layer F.Cu) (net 8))
 (segment (start 141.2 96.3) (end 141.7 96.3) (width 0.2) (layer F.Cu) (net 8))
 (segment (start 143.5 86.7) (end 143.5 86.05) (width 0.3048) (layer F.Cu) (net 10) (status C00030))
 (segment (start 143.5 86.05) (end 143.55 86) (width 0.3048) (layer F.Cu) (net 10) (status C00030))
 (segment (start 140.9 92.55) (end 140.9 91.5) (width 0.2) (layer F.Cu) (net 10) (status 400010))
 (segment (start 142.7 86.85) (end 143.55 86) (width 0.254) (layer F.Cu) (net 10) (status 800020))
 (segment (start 142.7 90.4) (end 142.7 86.85) (width 0.254) (layer F.Cu) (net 10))
 (segment (start 142.2 90.9) (end 142.7 90.4) (width 0.254) (layer F.Cu) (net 10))
 (segment (start 141.5 90.9) (end 142.2 90.9) (width 0.254) (layer F.Cu) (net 10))
 (segment (start 141.2 91.2) (end 141.5 90.9) (width 0.254) (layer F.Cu) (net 10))
 (segment (start 140.9 91.5) (end 141.2 91.2) (width 0.2) (layer F.Cu) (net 10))
 (segment (start 134.05 100) (end 134.1 100) (width 0.254) (layer F.Cu) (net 16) (status 30))
 (segment (start 134.1 100) (end 134.7 99.4) (width 0.254) (layer F.Cu) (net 16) (status 10))
 (segment (start 134.7 99.4) (end 134.7 97.7) (width 0.254) (layer F.Cu) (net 16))
 (segment (start 134.7 97.7) (end 135.5 96.9) (width 0.254) (layer F.Cu) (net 16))
 (segment (start 135.5 96.9) (end 135.7 96.7) (width 0.254) (layer F.Cu) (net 16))
 (segment (start 135.7 96.7) (end 139.2 96.7) (width 0.254) (layer F.Cu) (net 16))
 (segment (start 140.1 95.45) (end 140.1 96.1) (width 0.2) (layer F.Cu) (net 16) (status 10))
 (segment (start 139.5 96.7) (end 139.2 96.7) (width 0.2) (layer F.Cu) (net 16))
 (segment (start 140.1 96.1) (end 139.5 96.7) (width 0.2) (layer F.Cu) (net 16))
 (segment (start 140.5 95.45) (end 140.5 96.5) (width 0.2) (layer F.Cu) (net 6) (status 400010))
 (segment (start 143 100) (end 143.55 100) (width 0.254) (layer F.Cu) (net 6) (status 800020))
 (segment (start 142.3 99.3) (end 143 100) (width 0.254) (layer F.Cu) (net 6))
 (segment (start 142.3 97.7) (end 142.3 99.3) (width 0.254) (layer F.Cu) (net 6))
 (segment (start 141.4 96.8) (end 142.3 97.7) (width 0.254) (layer F.Cu) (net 6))
 (segment (start 140.8 96.8) (end 141.4 96.8) (width 0.254) (layer F.Cu) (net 6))
 (segment (start 140.5 96.5) (end 140.8 96.8) (width 0.254) (layer F.Cu) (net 6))
 (segment (start 143.5 87.3) (end 143.5 87.95) (width 0.3048) (layer F.Cu) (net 12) (status C00030))
 (segment (start 143.5 87.95) (end 143.55 88) (width 0.3048) (layer F.Cu) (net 12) (status C00030))
 (segment (start 141.3 92.55) (end 141.3 91.8) (width 0.2) (layer F.Cu) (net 12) (status 400010))
 (segment (start 143.4 88.15) (end 143.55 88) (width 0.254) (layer F.Cu) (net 12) (status C00030))
 (segment (start 143.4 90.5) (end 143.4 88.15) (width 0.254) (layer F.Cu) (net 12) (status 800020))
 (segment (start 142.3 91.6) (end 143.4 90.5) (width 0.254) (layer F.Cu) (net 12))
 (segment (start 141.7 91.6) (end 142.3 91.6) (width 0.254) (layer F.Cu) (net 12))
 (segment (start 141.3 91.8) (end 141.5 91.6) (width 0.2) (layer F.Cu) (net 12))
 (segment (start 141.5 91.6) (end 141.7 91.6) (width 0.2) (layer F.Cu) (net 12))
 (segment (start 139.7 92.55) (end 139.15 92.55) (width 0.2) (layer F.Cu) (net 23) (status 400010))
 (segment (start 137 86) (end 137.65 86) (width 0.254) (layer F.Cu) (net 23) (status C00030))
 (segment (start 136.2 86.8) (end 137 86) (width 0.254) (layer F.Cu) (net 23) (status 800020))
 (segment (start 136.2 90.3) (end 136.2 86.8) (width 0.254) (layer F.Cu) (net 23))
 (segment (start 138.8 92.2) (end 138.1 92.2) (width 0.254) (layer F.Cu) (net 23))
 (segment (start 139.15 92.55) (end 138.8 92.2) (width 0.2) (layer F.Cu) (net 23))
 (segment (start 138.1 92.2) (end 136.2 90.3) (width 0.254) (layer F.Cu) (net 23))
 (segment (start 137 95.95) (end 134.45 95.95) (width 0.254) (layer F.Cu) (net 17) (status 400010))
 (segment (start 137.3 96.3) (end 139 98) (width 0.254) (layer B.Cu) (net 17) (status 800020))
 (segment (start 134.3 96.3) (end 137.3 96.3) (width 0.254) (layer B.Cu) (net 17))
 (segment (start 134.2 96.2) (end 134.3 96.3) (width 0.254) (layer B.Cu) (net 17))
 (via (at 134.2 96.2) (size 0.6) (drill 0.4) (layers F.Cu B.Cu) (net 17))
 (segment (start 134.45 95.95) (end 134.2 96.2) (width 0.254) (layer F.Cu) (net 17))
 (segment (start 141.5 88.05) (end 141.5 87.15) (width 0.254) (layer F.Cu) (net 14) (status 400010))
 (segment (start 141.5 87.15) (end 140.35 86) (width 0.254) (layer F.Cu) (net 14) (status 800020))
 (segment (start 135.95 100) (end 137.65 100) (width 0.3048) (layer F.Cu) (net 15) (status C00030))
 (segment (start 134.45 86.85) (end 134.5 86.8) (width 0.3048) (layer F.Cu) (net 4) (status C00030))
 (segment (start 134.45 87.5) (end 134.45 86.85) (width 0.3048) (layer F.Cu) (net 4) (status C00030))
 (segment (start 134.45 87.5) (end 134.45 88.85) (width 0.254) (layer F.Cu) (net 4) (status 10))
 (segment (start 134.45 88.85) (end 133.3 90) (width 0.254) (layer F.Cu) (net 4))
 (segment (start 133.3 90) (end 133.3 93.7) (width 0.254) (layer F.Cu) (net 4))
 (segment (start 134.4 94.8) (end 134.9 94.8) (width 0.254) (layer F.Cu) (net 4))
 (segment (start 134.9 94.8) (end 134.918989 94.818989) (width 0.254) (layer F.Cu) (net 4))
 (segment (start 133.3 93.7) (end 134.4 94.8) (width 0.254) (layer F.Cu) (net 4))
 (segment (start 134.9 94.8) (end 137.6 94.8) (width 0.254) (layer F.Cu) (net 4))
 (segment (start 139.05 94.4) (end 138.1 94.4) (width 0.2) (layer F.Cu) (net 4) (status 10))
 (segment (start 137.7 94.8) (end 137.6 94.8) (width 0.2) (layer F.Cu) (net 4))
 (segment (start 138.1 94.4) (end 137.7 94.8) (width 0.2) (layer F.Cu) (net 4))
 (segment (start 132.9 98.3) (end 133.74599 98.3) (width 0.254) (layer F.Cu) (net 24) (status 30))
 (segment (start 133.9 98.3) (end 133.9 97.3) (width 0.254) (layer F.Cu) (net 24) (status 10))
 (segment (start 133.572999 95.899039) (end 134.199039 95.272999) (width 0.254) (layer F.Cu) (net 24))
 (segment (start 133.572999 96.972999) (end 133.572999 95.899039) (width 0.254) (layer F.Cu) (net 24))
 (segment (start 133.9 97.3) (end 133.572999 96.972999) (width 0.254) (layer F.Cu) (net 24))
 (segment (start 134.199039 95.272999) (end 136.088399 95.272999) (width 0.254) (layer F.Cu) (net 24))
 (segment (start 136.088399 95.272999) (end 137.7 95.272999) (width 0.254) (layer F.Cu) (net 24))
 (segment (start 137.827001 95.272999) (end 137.7 95.272999) (width 0.2) (layer F.Cu) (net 24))
 (segment (start 138.3 94.8) (end 137.827001 95.272999) (width 0.2) (layer F.Cu) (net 24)))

